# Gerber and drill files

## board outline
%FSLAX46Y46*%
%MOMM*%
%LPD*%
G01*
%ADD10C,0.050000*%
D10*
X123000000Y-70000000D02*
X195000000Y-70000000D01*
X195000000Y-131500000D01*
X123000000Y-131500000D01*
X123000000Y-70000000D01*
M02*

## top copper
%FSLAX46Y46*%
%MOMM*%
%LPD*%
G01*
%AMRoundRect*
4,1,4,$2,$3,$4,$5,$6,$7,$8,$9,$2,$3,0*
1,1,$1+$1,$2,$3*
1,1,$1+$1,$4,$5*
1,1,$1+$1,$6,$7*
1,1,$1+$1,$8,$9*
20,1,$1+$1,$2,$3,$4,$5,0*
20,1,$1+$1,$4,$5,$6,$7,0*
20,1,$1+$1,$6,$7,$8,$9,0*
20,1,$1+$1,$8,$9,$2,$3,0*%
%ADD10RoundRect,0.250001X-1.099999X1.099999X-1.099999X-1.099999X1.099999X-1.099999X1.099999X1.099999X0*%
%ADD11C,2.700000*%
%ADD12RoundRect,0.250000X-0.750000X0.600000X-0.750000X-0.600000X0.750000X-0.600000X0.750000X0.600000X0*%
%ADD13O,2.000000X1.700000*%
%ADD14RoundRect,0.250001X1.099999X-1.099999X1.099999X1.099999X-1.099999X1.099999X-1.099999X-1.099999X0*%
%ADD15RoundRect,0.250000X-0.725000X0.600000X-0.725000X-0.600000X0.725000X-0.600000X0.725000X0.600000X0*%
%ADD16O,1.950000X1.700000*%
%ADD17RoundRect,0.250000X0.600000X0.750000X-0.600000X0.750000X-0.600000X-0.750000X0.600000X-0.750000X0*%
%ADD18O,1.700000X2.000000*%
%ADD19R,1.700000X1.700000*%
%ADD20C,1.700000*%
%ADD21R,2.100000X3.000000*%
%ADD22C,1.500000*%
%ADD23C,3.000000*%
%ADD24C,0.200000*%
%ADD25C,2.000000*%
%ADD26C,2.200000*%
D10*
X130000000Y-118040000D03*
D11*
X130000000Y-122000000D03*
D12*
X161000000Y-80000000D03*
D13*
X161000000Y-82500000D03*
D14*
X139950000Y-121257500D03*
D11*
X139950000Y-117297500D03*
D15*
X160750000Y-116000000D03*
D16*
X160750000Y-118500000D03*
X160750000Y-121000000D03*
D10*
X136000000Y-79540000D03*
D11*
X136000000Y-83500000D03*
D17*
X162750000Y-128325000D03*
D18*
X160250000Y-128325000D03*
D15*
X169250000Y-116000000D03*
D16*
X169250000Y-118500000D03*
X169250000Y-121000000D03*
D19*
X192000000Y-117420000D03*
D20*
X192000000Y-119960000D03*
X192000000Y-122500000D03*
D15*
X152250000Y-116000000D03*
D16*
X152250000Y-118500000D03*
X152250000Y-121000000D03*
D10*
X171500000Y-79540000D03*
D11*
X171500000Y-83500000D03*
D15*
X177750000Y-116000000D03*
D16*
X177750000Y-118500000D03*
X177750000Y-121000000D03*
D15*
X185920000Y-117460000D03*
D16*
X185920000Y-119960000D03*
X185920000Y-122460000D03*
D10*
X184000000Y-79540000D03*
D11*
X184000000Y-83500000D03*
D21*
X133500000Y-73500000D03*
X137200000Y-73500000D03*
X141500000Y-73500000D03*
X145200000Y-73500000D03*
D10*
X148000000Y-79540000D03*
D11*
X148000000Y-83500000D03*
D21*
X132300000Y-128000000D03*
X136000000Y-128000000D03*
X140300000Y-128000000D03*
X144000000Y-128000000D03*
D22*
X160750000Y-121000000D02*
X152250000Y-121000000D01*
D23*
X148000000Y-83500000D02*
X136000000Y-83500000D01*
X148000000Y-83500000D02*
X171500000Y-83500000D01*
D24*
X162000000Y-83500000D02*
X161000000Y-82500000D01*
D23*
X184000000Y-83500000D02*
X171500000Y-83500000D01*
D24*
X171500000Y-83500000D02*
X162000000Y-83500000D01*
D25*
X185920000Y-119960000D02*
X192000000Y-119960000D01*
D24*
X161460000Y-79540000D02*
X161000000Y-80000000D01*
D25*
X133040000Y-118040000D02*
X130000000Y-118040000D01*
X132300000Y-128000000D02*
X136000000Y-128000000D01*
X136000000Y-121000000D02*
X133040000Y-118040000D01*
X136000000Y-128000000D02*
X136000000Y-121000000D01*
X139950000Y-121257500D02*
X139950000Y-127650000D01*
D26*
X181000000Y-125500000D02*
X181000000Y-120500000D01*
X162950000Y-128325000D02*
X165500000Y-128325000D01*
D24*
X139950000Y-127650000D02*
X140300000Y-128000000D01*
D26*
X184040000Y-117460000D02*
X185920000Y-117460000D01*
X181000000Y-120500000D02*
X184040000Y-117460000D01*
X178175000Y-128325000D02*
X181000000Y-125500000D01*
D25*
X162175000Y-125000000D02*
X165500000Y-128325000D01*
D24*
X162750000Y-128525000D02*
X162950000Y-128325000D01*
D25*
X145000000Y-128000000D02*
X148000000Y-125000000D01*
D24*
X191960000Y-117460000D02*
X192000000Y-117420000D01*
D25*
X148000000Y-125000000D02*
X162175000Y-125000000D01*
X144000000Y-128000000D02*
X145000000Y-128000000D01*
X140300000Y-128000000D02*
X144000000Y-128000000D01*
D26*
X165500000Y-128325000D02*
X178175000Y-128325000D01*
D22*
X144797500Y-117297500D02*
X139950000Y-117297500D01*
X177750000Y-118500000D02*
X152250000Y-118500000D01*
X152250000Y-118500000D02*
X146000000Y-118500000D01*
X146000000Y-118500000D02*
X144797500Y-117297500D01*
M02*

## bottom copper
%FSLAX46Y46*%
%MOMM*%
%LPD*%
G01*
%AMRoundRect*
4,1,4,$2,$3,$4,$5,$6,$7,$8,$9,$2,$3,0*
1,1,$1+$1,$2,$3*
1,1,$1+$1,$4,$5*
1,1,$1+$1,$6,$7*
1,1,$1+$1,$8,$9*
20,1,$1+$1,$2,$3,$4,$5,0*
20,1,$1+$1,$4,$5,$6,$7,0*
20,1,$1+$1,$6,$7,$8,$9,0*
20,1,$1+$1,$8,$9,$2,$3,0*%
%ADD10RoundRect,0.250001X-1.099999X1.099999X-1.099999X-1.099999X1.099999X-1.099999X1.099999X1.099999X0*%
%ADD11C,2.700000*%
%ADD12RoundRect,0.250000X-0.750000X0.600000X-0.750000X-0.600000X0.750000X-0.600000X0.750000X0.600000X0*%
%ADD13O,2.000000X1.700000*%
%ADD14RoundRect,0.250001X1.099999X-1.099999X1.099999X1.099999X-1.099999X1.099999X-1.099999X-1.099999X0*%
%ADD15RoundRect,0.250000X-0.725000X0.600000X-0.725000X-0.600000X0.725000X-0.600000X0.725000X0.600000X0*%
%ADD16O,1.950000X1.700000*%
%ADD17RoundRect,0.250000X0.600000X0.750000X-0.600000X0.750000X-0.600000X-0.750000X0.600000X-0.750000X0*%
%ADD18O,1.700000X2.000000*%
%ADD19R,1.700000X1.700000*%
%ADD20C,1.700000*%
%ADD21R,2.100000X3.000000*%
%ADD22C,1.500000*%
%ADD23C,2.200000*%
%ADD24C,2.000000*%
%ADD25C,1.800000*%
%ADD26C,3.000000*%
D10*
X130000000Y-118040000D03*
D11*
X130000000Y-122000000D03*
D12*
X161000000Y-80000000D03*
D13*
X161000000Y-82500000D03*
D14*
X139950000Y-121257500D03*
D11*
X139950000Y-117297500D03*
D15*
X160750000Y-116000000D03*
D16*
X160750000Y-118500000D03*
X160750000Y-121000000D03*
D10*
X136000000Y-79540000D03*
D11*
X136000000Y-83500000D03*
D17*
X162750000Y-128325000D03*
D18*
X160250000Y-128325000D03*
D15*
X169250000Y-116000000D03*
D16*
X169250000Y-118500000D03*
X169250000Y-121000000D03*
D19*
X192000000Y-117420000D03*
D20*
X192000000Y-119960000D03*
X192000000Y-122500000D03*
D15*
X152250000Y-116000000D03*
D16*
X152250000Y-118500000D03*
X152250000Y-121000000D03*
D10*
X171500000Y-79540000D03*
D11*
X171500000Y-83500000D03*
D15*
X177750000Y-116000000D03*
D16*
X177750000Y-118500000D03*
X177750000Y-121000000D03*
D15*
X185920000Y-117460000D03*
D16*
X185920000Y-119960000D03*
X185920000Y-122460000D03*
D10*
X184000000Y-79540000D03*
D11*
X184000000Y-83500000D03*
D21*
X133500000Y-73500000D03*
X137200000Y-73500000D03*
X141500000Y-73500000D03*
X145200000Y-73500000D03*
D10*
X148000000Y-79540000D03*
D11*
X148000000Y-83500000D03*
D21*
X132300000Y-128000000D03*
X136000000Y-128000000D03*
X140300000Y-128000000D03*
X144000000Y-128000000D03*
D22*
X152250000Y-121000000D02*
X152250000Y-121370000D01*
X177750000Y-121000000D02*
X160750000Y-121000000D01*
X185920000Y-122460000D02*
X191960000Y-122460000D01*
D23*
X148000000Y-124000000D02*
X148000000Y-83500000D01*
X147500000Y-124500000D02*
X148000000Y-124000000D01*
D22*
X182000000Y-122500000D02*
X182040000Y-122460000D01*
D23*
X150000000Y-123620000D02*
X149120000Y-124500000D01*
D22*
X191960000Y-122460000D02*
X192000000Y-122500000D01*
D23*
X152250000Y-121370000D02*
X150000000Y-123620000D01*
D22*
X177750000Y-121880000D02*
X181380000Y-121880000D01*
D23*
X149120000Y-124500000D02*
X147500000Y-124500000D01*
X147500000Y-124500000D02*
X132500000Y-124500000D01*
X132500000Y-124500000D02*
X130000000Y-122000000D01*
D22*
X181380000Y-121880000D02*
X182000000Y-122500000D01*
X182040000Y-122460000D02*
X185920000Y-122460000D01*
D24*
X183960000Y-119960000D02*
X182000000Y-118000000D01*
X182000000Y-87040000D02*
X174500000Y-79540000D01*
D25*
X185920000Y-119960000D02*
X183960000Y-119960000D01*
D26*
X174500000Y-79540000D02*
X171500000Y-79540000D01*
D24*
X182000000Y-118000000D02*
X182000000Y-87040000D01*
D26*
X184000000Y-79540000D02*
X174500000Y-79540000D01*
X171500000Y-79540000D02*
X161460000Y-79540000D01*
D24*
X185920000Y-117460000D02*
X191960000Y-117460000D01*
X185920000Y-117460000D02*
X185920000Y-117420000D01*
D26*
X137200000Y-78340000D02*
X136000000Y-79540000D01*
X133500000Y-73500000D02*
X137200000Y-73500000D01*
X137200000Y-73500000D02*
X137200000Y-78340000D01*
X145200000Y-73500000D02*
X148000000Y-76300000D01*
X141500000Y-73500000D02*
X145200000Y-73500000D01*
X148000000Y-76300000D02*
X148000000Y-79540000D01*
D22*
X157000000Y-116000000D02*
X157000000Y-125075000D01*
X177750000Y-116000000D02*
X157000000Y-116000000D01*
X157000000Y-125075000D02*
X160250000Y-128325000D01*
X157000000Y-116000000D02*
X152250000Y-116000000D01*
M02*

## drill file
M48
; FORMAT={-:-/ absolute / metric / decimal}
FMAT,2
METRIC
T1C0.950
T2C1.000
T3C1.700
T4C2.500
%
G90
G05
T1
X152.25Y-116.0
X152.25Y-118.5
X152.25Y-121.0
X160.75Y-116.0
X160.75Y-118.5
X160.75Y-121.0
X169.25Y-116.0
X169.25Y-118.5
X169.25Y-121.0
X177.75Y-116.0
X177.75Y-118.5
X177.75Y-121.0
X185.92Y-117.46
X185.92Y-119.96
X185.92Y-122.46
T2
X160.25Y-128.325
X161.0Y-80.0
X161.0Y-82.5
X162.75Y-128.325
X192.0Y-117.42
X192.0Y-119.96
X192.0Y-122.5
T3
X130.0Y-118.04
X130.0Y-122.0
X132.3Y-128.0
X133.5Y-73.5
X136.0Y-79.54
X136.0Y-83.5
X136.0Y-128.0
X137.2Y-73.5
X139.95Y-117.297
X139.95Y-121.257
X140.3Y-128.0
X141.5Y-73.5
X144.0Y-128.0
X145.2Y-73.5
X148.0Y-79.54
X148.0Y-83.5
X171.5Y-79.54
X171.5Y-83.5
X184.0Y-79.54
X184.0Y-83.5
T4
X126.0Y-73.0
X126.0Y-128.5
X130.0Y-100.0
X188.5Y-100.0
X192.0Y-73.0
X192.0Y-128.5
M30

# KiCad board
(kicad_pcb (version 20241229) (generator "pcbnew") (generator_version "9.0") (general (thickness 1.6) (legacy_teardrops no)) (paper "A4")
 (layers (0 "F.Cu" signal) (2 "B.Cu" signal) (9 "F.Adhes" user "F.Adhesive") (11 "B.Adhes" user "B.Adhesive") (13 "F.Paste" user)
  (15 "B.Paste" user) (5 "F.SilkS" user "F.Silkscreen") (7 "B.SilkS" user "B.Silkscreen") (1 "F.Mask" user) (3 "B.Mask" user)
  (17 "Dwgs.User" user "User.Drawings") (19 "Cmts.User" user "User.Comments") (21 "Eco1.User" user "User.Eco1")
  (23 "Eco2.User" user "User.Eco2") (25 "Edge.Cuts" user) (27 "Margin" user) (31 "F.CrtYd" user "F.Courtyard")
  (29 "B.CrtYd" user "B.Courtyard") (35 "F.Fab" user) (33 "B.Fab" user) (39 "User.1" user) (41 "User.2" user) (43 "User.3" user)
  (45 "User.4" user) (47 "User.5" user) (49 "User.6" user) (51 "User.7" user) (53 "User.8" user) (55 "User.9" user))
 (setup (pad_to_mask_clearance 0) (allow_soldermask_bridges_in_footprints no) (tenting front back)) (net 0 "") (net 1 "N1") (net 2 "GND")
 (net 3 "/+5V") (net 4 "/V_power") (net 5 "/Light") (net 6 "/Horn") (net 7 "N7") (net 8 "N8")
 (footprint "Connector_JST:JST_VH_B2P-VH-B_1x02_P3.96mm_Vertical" (layer "F.Cu") (at 130 118.04 -90)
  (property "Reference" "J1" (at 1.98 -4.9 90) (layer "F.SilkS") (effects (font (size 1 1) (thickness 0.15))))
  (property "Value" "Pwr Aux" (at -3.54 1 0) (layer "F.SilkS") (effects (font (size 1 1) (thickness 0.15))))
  (pad "1" thru_hole roundrect (at 0 0 270) (size 2.7 2.7) (drill 1.7) (layers "*.Cu" "*.Mask") (remove_unused_layers no)
   (roundrect_rratio 0.092593) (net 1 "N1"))
  (pad "2" thru_hole circle (at 3.96 0 270) (size 2.7 2.7) (drill 1.7) (layers "*.Cu" "*.Mask") (remove_unused_layers no) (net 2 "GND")))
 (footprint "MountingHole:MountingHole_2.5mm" (layer "F.Cu") (at 192 73)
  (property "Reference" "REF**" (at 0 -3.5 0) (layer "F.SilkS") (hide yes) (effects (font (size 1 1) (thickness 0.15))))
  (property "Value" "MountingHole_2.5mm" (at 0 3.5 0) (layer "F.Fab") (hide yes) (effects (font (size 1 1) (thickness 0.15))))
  (pad "" np_thru_hole circle (at 0 0) (size 2.5 2.5) (drill 2.5) (layers "*.Cu" "*.Mask")))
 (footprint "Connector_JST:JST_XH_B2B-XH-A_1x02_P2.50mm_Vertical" (layer "F.Cu") (at 161 80 -90)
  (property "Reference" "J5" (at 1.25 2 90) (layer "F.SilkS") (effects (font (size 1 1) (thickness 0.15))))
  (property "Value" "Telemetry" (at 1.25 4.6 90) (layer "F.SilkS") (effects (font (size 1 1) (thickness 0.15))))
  (pad "1" thru_hole roundrect (at 0 0 270) (size 1.7 2) (drill 1) (layers "*.Cu" "*.Mask") (remove_unused_layers no)
   (roundrect_rratio 0.147059) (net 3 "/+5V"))
  (pad "2" thru_hole oval (at 2.5 0 270) (size 1.7 2) (drill 1) (layers "*.Cu" "*.Mask") (remove_unused_layers no) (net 2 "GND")))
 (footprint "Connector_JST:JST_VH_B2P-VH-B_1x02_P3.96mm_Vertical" (layer "F.Cu") (at 139.95 121.2575 90)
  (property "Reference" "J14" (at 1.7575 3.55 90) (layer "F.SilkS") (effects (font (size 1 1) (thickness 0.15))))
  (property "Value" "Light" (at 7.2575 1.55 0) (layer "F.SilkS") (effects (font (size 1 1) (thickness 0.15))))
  (pad "1" thru_hole roundrect (at 0 0 90) (size 2.7 2.7) (drill 1.7) (layers "*.Cu" "*.Mask") (remove_unused_layers no)
   (roundrect_rratio 0.092593) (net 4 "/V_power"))
  (pad "2" thru_hole circle (at 3.96 0 90) (size 2.7 2.7) (drill 1.7) (layers "*.Cu" "*.Mask") (remove_unused_layers no) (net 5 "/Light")))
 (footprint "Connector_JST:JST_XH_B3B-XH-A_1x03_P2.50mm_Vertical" (layer "F.Cu") (at 160.75 116 -90)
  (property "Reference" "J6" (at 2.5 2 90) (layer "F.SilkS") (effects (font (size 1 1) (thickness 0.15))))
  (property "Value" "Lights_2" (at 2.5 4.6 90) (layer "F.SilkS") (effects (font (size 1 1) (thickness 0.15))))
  (pad "1" thru_hole roundrect (at 0 0 270) (size 1.7 1.95) (drill 0.95) (layers "*.Cu" "*.Mask") (remove_unused_layers no)
   (roundrect_rratio 0.147059) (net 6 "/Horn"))
  (pad "2" thru_hole oval (at 2.5 0 270) (size 1.7 1.95) (drill 0.95) (layers "*.Cu" "*.Mask") (remove_unused_layers no) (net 5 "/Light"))
  (pad "3" thru_hole oval (at 5 0 270) (size 1.7 1.95) (drill 0.95) (layers "*.Cu" "*.Mask") (remove_unused_layers no) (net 2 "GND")))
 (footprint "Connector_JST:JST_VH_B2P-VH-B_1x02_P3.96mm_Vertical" (layer "F.Cu") (at 136 79.54 -90)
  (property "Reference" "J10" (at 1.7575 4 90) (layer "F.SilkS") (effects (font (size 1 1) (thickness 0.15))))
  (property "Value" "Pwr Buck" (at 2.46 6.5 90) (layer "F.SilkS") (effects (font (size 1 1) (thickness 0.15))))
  (pad "1" thru_hole roundrect (at 0 0 270) (size 2.7 2.7) (drill 1.7) (layers "*.Cu" "*.Mask") (remove_unused_layers no)
   (roundrect_rratio 0.092593) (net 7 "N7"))
  (pad "2" thru_hole circle (at 3.96 0 270) (size 2.7 2.7) (drill 1.7) (layers "*.Cu" "*.Mask") (remove_unused_layers no) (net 2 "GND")))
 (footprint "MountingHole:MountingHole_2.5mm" (layer "F.Cu") (at 130 100)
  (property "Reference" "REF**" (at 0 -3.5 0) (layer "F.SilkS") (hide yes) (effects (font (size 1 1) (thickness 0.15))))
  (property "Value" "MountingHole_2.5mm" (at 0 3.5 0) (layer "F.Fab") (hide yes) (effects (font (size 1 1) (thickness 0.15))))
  (pad "" np_thru_hole circle (at 0 0) (size 2.5 2.5) (drill 2.5) (layers "*.Cu" "*.Mask")))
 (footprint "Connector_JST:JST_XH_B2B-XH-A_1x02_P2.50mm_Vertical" (layer "F.Cu") (at 162.75 128.325 180)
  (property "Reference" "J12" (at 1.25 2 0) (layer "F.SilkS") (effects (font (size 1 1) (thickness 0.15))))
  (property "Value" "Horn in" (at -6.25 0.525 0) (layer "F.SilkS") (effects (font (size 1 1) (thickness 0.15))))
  (pad "1" thru_hole roundrect (at 0 0 180) (size 1.7 2) (drill 1) (layers "*.Cu" "*.Mask") (remove_unused_layers no)
   (roundrect_rratio 0.147059) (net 4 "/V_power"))
  (pad "2" thru_hole oval (at 2.5 0 180) (size 1.7 2) (drill 1) (layers "*.Cu" "*.Mask") (remove_unused_layers no) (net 6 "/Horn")))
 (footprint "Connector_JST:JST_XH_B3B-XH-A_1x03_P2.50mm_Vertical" (layer "F.Cu") (at 169.25 116 -90)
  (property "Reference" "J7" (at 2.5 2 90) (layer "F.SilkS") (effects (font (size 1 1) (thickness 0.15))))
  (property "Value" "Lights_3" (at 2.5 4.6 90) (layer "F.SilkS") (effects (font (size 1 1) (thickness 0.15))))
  (pad "1" thru_hole roundrect (at 0 0 270) (size 1.7 1.95) (drill 0.95) (layers "*.Cu" "*.Mask") (remove_unused_layers no)
   (roundrect_rratio 0.147059) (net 6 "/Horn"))
  (pad "2" thru_hole oval (at 2.5 0 270) (size 1.7 1.95) (drill 0.95) (layers "*.Cu" "*.Mask") (remove_unused_layers no) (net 5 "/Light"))
  (pad "3" thru_hole oval (at 5 0 270) (size 1.7 1.95) (drill 0.95) (layers "*.Cu" "*.Mask") (remove_unused_layers no) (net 2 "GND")))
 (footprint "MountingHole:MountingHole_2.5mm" (layer "F.Cu") (at 188.5 100)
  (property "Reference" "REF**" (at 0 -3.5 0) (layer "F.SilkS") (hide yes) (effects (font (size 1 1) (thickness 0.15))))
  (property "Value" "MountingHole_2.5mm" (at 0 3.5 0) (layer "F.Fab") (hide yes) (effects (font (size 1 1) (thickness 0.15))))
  (pad "" np_thru_hole circle (at 0 0) (size 2.5 2.5) (drill 2.5) (layers "*.Cu" "*.Mask")))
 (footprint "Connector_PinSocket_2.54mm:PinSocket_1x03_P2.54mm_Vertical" (layer "F.Cu") (at 192 117.42)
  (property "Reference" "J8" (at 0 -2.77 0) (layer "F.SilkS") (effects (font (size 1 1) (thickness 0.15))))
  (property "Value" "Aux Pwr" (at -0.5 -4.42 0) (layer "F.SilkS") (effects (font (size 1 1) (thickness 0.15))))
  (pad "1" thru_hole rect (at 0 0) (size 1.7 1.7) (drill 1) (layers "*.Cu" "*.Mask") (remove_unused_layers no) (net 4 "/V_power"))
  (pad "2" thru_hole circle (at 0 2.54) (size 1.7 1.7) (drill 1) (layers "*.Cu" "*.Mask") (remove_unused_layers no) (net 3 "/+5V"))
  (pad "3" thru_hole circle (at 0 5.08) (size 1.7 1.7) (drill 1) (layers "*.Cu" "*.Mask") (remove_unused_layers no) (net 2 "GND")))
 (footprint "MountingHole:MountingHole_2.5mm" (layer "F.Cu") (at 126 73)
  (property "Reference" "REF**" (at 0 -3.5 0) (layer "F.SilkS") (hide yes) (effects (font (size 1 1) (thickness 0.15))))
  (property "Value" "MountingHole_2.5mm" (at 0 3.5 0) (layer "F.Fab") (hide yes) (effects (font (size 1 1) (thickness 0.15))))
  (pad "" np_thru_hole circle (at 0 0) (size 2.5 2.5) (drill 2.5) (layers "*.Cu" "*.Mask")))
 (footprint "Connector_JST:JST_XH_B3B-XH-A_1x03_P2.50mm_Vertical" (layer "F.Cu") (at 152.25 116 -90)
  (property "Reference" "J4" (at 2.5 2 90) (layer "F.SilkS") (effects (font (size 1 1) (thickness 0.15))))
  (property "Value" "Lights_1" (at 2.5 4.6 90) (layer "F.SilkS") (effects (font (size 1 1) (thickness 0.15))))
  (pad "1" thru_hole roundrect (at 0 0 270) (size 1.7 1.95) (drill 0.95) (layers "*.Cu" "*.Mask") (remove_unused_layers no)
   (roundrect_rratio 0.147059) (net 6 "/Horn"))
  (pad "2" thru_hole oval (at 2.5 0 270) (size 1.7 1.95) (drill 0.95) (layers "*.Cu" "*.Mask") (remove_unused_layers no) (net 5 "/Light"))
  (pad "3" thru_hole oval (at 5 0 270) (size 1.7 1.95) (drill 0.95) (layers "*.Cu" "*.Mask") (remove_unused_layers no) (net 2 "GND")))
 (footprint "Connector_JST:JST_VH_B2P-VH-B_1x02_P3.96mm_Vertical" (layer "F.Cu") (at 171.5 79.54 -90)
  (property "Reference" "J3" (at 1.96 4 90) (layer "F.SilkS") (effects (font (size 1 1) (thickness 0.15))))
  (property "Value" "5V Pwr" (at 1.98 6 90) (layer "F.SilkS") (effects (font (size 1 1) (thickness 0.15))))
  (pad "1" thru_hole roundrect (at 0 0 270) (size 2.7 2.7) (drill 1.7) (layers "*.Cu" "*.Mask") (remove_unused_layers no)
   (roundrect_rratio 0.092593) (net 3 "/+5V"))
  (pad "2" thru_hole circle (at 3.96 0 270) (size 2.7 2.7) (drill 1.7) (layers "*.Cu" "*.Mask") (remove_unused_layers no) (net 2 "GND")))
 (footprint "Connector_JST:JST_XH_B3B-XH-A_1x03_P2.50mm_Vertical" (layer "F.Cu") (at 177.75 116 -90)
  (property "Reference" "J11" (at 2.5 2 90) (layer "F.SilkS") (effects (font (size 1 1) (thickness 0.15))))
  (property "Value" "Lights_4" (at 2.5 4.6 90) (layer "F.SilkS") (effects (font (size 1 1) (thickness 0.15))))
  (pad "1" thru_hole roundrect (at 0 0 270) (size 1.7 1.95) (drill 0.95) (layers "*.Cu" "*.Mask") (remove_unused_layers no)
   (roundrect_rratio 0.147059) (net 6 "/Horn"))
  (pad "2" thru_hole oval (at 2.5 0 270) (size 1.7 1.95) (drill 0.95) (layers "*.Cu" "*.Mask") (remove_unused_layers no) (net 5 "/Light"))
  (pad "3" thru_hole oval (at 5 0 270) (size 1.7 1.95) (drill 0.95) (layers "*.Cu" "*.Mask") (remove_unused_layers no) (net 2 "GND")))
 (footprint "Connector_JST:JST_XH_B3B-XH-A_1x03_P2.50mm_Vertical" (layer "F.Cu") (at 185.92 117.46 -90)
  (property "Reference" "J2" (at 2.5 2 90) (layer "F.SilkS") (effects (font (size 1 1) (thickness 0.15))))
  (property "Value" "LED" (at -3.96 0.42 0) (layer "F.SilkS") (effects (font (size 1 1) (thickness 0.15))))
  (pad "1" thru_hole roundrect (at 0 0 270) (size 1.7 1.95) (drill 0.95) (layers "*.Cu" "*.Mask") (remove_unused_layers no)
   (roundrect_rratio 0.147059) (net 4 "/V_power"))
  (pad "2" thru_hole oval (at 2.5 0 270) (size 1.7 1.95) (drill 0.95) (layers "*.Cu" "*.Mask") (remove_unused_layers no) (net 3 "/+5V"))
  (pad "3" thru_hole oval (at 5 0 270) (size 1.7 1.95) (drill 0.95) (layers "*.Cu" "*.Mask") (remove_unused_layers no) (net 2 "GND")))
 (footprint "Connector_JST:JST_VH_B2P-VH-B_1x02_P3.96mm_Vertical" (layer "F.Cu") (at 184 79.54 -90)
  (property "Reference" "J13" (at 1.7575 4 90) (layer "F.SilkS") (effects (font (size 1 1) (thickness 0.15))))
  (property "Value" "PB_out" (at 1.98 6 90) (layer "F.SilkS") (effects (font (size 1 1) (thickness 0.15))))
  (pad "1" thru_hole roundrect (at 0 0 270) (size 2.7 2.7) (drill 1.7) (layers "*.Cu" "*.Mask") (remove_unused_layers no)
   (roundrect_rratio 0.092593) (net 3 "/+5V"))
  (pad "2" thru_hole circle (at 3.96 0 270) (size 2.7 2.7) (drill 1.7) (layers "*.Cu" "*.Mask") (remove_unused_layers no) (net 2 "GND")))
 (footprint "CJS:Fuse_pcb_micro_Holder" (layer "F.Cu") (at 139.35 73.5)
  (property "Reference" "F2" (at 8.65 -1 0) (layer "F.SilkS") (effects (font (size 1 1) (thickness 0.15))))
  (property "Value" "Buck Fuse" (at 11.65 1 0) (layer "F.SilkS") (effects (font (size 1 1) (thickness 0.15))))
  (pad "1" thru_hole rect (at -5.85 0) (size 2.1 3) (drill 1.7) (layers "*.Cu" "*.Mask") (remove_unused_layers no) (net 7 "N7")
   (thermal_bridge_angle 45))
  (pad "2" thru_hole rect (at -2.15 0) (size 2.1 3) (drill 1.7) (layers "*.Cu" "*.Mask") (remove_unused_layers no) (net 7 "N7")
   (thermal_bridge_angle 45))
  (pad "3" thru_hole rect (at 2.15 0) (size 2.1 3) (drill 1.7) (layers "*.Cu" "*.Mask") (remove_unused_layers no) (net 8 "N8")
   (thermal_bridge_angle 45))
  (pad "4" thru_hole rect (at 5.85 0) (size 2.1 3) (drill 1.7) (layers "*.Cu" "*.Mask") (remove_unused_layers no) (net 8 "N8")
   (thermal_bridge_angle 45)))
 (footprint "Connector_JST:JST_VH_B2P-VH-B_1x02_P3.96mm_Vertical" (layer "F.Cu") (at 148 79.54 -90)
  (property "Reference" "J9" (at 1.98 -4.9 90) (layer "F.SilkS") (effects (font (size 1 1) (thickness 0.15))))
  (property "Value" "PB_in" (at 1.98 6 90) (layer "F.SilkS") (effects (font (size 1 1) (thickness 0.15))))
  (pad "1" thru_hole roundrect (at 0 0 270) (size 2.7 2.7) (drill 1.7) (layers "*.Cu" "*.Mask") (remove_unused_layers no)
   (roundrect_rratio 0.092593) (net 8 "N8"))
  (pad "2" thru_hole circle (at 3.96 0 270) (size 2.7 2.7) (drill 1.7) (layers "*.Cu" "*.Mask") (remove_unused_layers no) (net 2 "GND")))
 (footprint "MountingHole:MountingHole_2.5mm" (layer "F.Cu") (at 192 128.5)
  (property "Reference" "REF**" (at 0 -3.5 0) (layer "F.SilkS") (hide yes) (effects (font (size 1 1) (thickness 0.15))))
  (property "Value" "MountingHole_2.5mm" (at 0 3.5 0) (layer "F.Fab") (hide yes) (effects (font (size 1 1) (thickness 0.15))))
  (pad "" np_thru_hole circle (at 0 0) (size 2.5 2.5) (drill 2.5) (layers "*.Cu" "*.Mask")))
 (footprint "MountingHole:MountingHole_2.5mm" (layer "F.Cu") (at 126 128.5)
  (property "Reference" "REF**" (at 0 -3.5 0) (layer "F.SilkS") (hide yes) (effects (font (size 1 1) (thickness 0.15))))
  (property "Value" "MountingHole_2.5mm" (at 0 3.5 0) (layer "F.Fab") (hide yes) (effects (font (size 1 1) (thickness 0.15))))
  (pad "" np_thru_hole circle (at 0 0) (size 2.5 2.5) (drill 2.5) (layers "*.Cu" "*.Mask")))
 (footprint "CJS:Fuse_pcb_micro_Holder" (layer "F.Cu") (at 138.15 128)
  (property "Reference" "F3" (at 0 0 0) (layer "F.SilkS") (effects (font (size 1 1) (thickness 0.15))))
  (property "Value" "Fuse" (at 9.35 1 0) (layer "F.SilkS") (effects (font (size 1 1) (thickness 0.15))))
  (pad "1" thru_hole rect (at -5.85 0) (size 2.1 3) (drill 1.7) (layers "*.Cu" "*.Mask") (remove_unused_layers no) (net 1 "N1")
   (thermal_bridge_angle 45))
  (pad "2" thru_hole rect (at -2.15 0) (size 2.1 3) (drill 1.7) (layers "*.Cu" "*.Mask") (remove_unused_layers no) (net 1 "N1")
   (thermal_bridge_angle 45))
  (pad "3" thru_hole rect (at 2.15 0) (size 2.1 3) (drill 1.7) (layers "*.Cu" "*.Mask") (remove_unused_layers no) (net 4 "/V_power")
   (thermal_bridge_angle 45))
  (pad "4" thru_hole rect (at 5.85 0) (size 2.1 3) (drill 1.7) (layers "*.Cu" "*.Mask") (remove_unused_layers no) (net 4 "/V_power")
   (thermal_bridge_angle 45)))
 (gr_rect (start 123 70) (end 195 131.5) (stroke (width 0.05) (type default)) (fill no) (layer "Edge.Cuts"))
 (segment (start 160.75 121) (end 152.25 121) (width 1.5) (layer "F.Cu") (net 2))
 (segment (start 148 83.5) (end 136 83.5) (width 3) (layer "F.Cu") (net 2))
 (segment (start 148 83.5) (end 171.5 83.5) (width 3) (layer "F.Cu") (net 2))
 (segment (start 162 83.5) (end 161 82.5) (width 0.2) (layer "F.Cu") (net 2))
 (segment (start 184 83.5) (end 171.5 83.5) (width 3) (layer "F.Cu") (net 2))
 (segment (start 171.5 83.5) (end 162 83.5) (width 0.2) (layer "F.Cu") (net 2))
 (segment (start 152.25 121) (end 152.25 121.37) (width 1.5) (layer "B.Cu") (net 2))
 (segment (start 177.75 121) (end 160.75 121) (width 1.5) (layer "B.Cu") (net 2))
 (segment (start 185.92 122.46) (end 191.96 122.46) (width 1.5) (layer "B.Cu") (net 2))
 (segment (start 148 124) (end 148 83.5) (width 2.2) (layer "B.Cu") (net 2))
 (segment (start 147.5 124.5) (end 148 124) (width 2.2) (layer "B.Cu") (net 2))
 (segment (start 182 122.5) (end 182.04 122.46) (width 1.5) (layer "B.Cu") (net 2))
 (segment (start 150 123.62) (end 149.12 124.5) (width 2.2) (layer "B.Cu") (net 2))
 (segment (start 191.96 122.46) (end 192 122.5) (width 1.5) (layer "B.Cu") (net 2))
 (segment (start 152.25 121.37) (end 150 123.62) (width 2.2) (layer "B.Cu") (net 2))
 (segment (start 177.75 121.88) (end 181.38 121.88) (width 1.5) (layer "B.Cu") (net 2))
 (segment (start 149.12 124.5) (end 147.5 124.5) (width 2.2) (layer "B.Cu") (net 2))
 (segment (start 147.5 124.5) (end 132.5 124.5) (width 2.2) (layer "B.Cu") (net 2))
 (segment (start 132.5 124.5) (end 130 122) (width 2.2) (layer "B.Cu") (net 2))
 (segment (start 181.38 121.88) (end 182 122.5) (width 1.5) (layer "B.Cu") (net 2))
 (segment (start 182.04 122.46) (end 185.92 122.46) (width 1.5) (layer "B.Cu") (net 2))
 (segment (start 185.92 119.96) (end 192 119.96) (width 2) (layer "F.Cu") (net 3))
 (segment (start 161.46 79.54) (end 161 80) (width 0.2) (layer "F.Cu") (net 3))
 (segment (start 183.96 119.96) (end 182 118) (width 2) (layer "B.Cu") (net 3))
 (segment (start 182 87.04) (end 174.5 79.54) (width 2) (layer "B.Cu") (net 3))
 (segment (start 185.92 119.96) (end 183.96 119.96) (width 1.8) (layer "B.Cu") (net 3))
 (segment (start 174.5 79.54) (end 171.5 79.54) (width 3) (layer "B.Cu") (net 3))
 (segment (start 182 118) (end 182 87.04) (width 2) (layer "B.Cu") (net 3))
 (segment (start 184 79.54) (end 174.5 79.54) (width 3) (layer "B.Cu") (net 3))
 (segment (start 171.5 79.54) (end 161.46 79.54) (width 3) (layer "B.Cu") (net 3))
 (segment (start 133.04 118.04) (end 130 118.04) (width 2) (layer "F.Cu") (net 1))
 (segment (start 132.3 128) (end 136 128) (width 2) (layer "F.Cu") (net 1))
 (segment (start 136 121) (end 133.04 118.04) (width 2) (layer "F.Cu") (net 1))
 (segment (start 136 128) (end 136 121) (width 2) (layer "F.Cu") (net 1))
 (segment (start 139.95 121.2575) (end 139.95 127.65) (width 2) (layer "F.Cu") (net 4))
 (segment (start 181 125.5) (end 181 120.5) (width 2.2) (layer "F.Cu") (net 4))
 (segment (start 162.95 128.325) (end 165.5 128.325) (width 2.2) (layer "F.Cu") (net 4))
 (segment (start 139.95 127.65) (end 140.3 128) (width 0.2) (layer "F.Cu") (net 4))
 (segment (start 184.04 117.46) (end 185.92 117.46) (width 2.2) (layer "F.Cu") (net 4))
 (segment (start 181 120.5) (end 184.04 117.46) (width 2.2) (layer "F.Cu") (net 4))
 (segment (start 178.175 128.325) (end 181 125.5) (width 2.2) (layer "F.Cu") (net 4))
 (segment (start 162.175 125) (end 165.5 128.325) (width 2) (layer "F.Cu") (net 4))
 (segment (start 162.75 128.525) (end 162.95 128.325) (width 0.2) (layer "F.Cu") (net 4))
 (segment (start 145 128) (end 148 125) (width 2) (layer "F.Cu") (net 4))
 (segment (start 191.96 117.46) (end 192 117.42) (width 0.2) (layer "F.Cu") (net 4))
 (segment (start 148 125) (end 162.175 125) (width 2) (layer "F.Cu") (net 4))
 (segment (start 144 128) (end 145 128) (width 2) (layer "F.Cu") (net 4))
 (segment (start 140.3 128) (end 144 128) (width 2) (layer "F.Cu") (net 4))
 (segment (start 165.5 128.325) (end 178.175 128.325) (width 2.2) (layer "F.Cu") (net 4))
 (segment (start 185.92 117.46) (end 191.96 117.46) (width 2) (layer "B.Cu") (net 4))
 (segment (start 185.92 117.46) (end 185.92 117.42) (width 2) (layer "B.Cu") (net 4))
 (segment (start 137.2 78.34) (end 136 79.54) (width 3) (layer "B.Cu") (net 7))
 (segment (start 133.5 73.5) (end 137.2 73.5) (width 3) (layer "B.Cu") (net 7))
 (segment (start 137.2 73.5) (end 137.2 78.34) (width 3) (layer "B.Cu") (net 7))
 (segment (start 145.2 73.5) (end 148 76.3) (width 3) (layer "B.Cu") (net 8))
 (segment (start 141.5 73.5) (end 145.2 73.5) (width 3) (layer "B.Cu") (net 8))
 (segment (start 148 76.3) (end 148 79.54) (width 3) (layer "B.Cu") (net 8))
 (segment (start 157 116) (end 157 125.075) (width 1.5) (layer "B.Cu") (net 6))
 (segment (start 177.75 116) (end 157 116) (width 1.5) (layer "B.Cu") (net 6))
 (segment (start 157 125.075) (end 160.25 128.325) (width 1.5) (layer "B.Cu") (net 6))
 (segment (start 157 116) (end 152.25 116) (width 1.5) (layer "B.Cu") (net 6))
 (segment (start 144.7975 117.2975) (end 139.95 117.2975) (width 1.5) (layer "F.Cu") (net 5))
 (segment (start 177.75 118.5) (end 152.25 118.5) (width 1.5) (layer "F.Cu") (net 5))
 (segment (start 152.25 118.5) (end 146 118.5) (width 1.5) (layer "F.Cu") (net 5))
 (segment (start 146 118.5) (end 144.7975 117.2975) (width 1.5) (layer "F.Cu") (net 5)))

